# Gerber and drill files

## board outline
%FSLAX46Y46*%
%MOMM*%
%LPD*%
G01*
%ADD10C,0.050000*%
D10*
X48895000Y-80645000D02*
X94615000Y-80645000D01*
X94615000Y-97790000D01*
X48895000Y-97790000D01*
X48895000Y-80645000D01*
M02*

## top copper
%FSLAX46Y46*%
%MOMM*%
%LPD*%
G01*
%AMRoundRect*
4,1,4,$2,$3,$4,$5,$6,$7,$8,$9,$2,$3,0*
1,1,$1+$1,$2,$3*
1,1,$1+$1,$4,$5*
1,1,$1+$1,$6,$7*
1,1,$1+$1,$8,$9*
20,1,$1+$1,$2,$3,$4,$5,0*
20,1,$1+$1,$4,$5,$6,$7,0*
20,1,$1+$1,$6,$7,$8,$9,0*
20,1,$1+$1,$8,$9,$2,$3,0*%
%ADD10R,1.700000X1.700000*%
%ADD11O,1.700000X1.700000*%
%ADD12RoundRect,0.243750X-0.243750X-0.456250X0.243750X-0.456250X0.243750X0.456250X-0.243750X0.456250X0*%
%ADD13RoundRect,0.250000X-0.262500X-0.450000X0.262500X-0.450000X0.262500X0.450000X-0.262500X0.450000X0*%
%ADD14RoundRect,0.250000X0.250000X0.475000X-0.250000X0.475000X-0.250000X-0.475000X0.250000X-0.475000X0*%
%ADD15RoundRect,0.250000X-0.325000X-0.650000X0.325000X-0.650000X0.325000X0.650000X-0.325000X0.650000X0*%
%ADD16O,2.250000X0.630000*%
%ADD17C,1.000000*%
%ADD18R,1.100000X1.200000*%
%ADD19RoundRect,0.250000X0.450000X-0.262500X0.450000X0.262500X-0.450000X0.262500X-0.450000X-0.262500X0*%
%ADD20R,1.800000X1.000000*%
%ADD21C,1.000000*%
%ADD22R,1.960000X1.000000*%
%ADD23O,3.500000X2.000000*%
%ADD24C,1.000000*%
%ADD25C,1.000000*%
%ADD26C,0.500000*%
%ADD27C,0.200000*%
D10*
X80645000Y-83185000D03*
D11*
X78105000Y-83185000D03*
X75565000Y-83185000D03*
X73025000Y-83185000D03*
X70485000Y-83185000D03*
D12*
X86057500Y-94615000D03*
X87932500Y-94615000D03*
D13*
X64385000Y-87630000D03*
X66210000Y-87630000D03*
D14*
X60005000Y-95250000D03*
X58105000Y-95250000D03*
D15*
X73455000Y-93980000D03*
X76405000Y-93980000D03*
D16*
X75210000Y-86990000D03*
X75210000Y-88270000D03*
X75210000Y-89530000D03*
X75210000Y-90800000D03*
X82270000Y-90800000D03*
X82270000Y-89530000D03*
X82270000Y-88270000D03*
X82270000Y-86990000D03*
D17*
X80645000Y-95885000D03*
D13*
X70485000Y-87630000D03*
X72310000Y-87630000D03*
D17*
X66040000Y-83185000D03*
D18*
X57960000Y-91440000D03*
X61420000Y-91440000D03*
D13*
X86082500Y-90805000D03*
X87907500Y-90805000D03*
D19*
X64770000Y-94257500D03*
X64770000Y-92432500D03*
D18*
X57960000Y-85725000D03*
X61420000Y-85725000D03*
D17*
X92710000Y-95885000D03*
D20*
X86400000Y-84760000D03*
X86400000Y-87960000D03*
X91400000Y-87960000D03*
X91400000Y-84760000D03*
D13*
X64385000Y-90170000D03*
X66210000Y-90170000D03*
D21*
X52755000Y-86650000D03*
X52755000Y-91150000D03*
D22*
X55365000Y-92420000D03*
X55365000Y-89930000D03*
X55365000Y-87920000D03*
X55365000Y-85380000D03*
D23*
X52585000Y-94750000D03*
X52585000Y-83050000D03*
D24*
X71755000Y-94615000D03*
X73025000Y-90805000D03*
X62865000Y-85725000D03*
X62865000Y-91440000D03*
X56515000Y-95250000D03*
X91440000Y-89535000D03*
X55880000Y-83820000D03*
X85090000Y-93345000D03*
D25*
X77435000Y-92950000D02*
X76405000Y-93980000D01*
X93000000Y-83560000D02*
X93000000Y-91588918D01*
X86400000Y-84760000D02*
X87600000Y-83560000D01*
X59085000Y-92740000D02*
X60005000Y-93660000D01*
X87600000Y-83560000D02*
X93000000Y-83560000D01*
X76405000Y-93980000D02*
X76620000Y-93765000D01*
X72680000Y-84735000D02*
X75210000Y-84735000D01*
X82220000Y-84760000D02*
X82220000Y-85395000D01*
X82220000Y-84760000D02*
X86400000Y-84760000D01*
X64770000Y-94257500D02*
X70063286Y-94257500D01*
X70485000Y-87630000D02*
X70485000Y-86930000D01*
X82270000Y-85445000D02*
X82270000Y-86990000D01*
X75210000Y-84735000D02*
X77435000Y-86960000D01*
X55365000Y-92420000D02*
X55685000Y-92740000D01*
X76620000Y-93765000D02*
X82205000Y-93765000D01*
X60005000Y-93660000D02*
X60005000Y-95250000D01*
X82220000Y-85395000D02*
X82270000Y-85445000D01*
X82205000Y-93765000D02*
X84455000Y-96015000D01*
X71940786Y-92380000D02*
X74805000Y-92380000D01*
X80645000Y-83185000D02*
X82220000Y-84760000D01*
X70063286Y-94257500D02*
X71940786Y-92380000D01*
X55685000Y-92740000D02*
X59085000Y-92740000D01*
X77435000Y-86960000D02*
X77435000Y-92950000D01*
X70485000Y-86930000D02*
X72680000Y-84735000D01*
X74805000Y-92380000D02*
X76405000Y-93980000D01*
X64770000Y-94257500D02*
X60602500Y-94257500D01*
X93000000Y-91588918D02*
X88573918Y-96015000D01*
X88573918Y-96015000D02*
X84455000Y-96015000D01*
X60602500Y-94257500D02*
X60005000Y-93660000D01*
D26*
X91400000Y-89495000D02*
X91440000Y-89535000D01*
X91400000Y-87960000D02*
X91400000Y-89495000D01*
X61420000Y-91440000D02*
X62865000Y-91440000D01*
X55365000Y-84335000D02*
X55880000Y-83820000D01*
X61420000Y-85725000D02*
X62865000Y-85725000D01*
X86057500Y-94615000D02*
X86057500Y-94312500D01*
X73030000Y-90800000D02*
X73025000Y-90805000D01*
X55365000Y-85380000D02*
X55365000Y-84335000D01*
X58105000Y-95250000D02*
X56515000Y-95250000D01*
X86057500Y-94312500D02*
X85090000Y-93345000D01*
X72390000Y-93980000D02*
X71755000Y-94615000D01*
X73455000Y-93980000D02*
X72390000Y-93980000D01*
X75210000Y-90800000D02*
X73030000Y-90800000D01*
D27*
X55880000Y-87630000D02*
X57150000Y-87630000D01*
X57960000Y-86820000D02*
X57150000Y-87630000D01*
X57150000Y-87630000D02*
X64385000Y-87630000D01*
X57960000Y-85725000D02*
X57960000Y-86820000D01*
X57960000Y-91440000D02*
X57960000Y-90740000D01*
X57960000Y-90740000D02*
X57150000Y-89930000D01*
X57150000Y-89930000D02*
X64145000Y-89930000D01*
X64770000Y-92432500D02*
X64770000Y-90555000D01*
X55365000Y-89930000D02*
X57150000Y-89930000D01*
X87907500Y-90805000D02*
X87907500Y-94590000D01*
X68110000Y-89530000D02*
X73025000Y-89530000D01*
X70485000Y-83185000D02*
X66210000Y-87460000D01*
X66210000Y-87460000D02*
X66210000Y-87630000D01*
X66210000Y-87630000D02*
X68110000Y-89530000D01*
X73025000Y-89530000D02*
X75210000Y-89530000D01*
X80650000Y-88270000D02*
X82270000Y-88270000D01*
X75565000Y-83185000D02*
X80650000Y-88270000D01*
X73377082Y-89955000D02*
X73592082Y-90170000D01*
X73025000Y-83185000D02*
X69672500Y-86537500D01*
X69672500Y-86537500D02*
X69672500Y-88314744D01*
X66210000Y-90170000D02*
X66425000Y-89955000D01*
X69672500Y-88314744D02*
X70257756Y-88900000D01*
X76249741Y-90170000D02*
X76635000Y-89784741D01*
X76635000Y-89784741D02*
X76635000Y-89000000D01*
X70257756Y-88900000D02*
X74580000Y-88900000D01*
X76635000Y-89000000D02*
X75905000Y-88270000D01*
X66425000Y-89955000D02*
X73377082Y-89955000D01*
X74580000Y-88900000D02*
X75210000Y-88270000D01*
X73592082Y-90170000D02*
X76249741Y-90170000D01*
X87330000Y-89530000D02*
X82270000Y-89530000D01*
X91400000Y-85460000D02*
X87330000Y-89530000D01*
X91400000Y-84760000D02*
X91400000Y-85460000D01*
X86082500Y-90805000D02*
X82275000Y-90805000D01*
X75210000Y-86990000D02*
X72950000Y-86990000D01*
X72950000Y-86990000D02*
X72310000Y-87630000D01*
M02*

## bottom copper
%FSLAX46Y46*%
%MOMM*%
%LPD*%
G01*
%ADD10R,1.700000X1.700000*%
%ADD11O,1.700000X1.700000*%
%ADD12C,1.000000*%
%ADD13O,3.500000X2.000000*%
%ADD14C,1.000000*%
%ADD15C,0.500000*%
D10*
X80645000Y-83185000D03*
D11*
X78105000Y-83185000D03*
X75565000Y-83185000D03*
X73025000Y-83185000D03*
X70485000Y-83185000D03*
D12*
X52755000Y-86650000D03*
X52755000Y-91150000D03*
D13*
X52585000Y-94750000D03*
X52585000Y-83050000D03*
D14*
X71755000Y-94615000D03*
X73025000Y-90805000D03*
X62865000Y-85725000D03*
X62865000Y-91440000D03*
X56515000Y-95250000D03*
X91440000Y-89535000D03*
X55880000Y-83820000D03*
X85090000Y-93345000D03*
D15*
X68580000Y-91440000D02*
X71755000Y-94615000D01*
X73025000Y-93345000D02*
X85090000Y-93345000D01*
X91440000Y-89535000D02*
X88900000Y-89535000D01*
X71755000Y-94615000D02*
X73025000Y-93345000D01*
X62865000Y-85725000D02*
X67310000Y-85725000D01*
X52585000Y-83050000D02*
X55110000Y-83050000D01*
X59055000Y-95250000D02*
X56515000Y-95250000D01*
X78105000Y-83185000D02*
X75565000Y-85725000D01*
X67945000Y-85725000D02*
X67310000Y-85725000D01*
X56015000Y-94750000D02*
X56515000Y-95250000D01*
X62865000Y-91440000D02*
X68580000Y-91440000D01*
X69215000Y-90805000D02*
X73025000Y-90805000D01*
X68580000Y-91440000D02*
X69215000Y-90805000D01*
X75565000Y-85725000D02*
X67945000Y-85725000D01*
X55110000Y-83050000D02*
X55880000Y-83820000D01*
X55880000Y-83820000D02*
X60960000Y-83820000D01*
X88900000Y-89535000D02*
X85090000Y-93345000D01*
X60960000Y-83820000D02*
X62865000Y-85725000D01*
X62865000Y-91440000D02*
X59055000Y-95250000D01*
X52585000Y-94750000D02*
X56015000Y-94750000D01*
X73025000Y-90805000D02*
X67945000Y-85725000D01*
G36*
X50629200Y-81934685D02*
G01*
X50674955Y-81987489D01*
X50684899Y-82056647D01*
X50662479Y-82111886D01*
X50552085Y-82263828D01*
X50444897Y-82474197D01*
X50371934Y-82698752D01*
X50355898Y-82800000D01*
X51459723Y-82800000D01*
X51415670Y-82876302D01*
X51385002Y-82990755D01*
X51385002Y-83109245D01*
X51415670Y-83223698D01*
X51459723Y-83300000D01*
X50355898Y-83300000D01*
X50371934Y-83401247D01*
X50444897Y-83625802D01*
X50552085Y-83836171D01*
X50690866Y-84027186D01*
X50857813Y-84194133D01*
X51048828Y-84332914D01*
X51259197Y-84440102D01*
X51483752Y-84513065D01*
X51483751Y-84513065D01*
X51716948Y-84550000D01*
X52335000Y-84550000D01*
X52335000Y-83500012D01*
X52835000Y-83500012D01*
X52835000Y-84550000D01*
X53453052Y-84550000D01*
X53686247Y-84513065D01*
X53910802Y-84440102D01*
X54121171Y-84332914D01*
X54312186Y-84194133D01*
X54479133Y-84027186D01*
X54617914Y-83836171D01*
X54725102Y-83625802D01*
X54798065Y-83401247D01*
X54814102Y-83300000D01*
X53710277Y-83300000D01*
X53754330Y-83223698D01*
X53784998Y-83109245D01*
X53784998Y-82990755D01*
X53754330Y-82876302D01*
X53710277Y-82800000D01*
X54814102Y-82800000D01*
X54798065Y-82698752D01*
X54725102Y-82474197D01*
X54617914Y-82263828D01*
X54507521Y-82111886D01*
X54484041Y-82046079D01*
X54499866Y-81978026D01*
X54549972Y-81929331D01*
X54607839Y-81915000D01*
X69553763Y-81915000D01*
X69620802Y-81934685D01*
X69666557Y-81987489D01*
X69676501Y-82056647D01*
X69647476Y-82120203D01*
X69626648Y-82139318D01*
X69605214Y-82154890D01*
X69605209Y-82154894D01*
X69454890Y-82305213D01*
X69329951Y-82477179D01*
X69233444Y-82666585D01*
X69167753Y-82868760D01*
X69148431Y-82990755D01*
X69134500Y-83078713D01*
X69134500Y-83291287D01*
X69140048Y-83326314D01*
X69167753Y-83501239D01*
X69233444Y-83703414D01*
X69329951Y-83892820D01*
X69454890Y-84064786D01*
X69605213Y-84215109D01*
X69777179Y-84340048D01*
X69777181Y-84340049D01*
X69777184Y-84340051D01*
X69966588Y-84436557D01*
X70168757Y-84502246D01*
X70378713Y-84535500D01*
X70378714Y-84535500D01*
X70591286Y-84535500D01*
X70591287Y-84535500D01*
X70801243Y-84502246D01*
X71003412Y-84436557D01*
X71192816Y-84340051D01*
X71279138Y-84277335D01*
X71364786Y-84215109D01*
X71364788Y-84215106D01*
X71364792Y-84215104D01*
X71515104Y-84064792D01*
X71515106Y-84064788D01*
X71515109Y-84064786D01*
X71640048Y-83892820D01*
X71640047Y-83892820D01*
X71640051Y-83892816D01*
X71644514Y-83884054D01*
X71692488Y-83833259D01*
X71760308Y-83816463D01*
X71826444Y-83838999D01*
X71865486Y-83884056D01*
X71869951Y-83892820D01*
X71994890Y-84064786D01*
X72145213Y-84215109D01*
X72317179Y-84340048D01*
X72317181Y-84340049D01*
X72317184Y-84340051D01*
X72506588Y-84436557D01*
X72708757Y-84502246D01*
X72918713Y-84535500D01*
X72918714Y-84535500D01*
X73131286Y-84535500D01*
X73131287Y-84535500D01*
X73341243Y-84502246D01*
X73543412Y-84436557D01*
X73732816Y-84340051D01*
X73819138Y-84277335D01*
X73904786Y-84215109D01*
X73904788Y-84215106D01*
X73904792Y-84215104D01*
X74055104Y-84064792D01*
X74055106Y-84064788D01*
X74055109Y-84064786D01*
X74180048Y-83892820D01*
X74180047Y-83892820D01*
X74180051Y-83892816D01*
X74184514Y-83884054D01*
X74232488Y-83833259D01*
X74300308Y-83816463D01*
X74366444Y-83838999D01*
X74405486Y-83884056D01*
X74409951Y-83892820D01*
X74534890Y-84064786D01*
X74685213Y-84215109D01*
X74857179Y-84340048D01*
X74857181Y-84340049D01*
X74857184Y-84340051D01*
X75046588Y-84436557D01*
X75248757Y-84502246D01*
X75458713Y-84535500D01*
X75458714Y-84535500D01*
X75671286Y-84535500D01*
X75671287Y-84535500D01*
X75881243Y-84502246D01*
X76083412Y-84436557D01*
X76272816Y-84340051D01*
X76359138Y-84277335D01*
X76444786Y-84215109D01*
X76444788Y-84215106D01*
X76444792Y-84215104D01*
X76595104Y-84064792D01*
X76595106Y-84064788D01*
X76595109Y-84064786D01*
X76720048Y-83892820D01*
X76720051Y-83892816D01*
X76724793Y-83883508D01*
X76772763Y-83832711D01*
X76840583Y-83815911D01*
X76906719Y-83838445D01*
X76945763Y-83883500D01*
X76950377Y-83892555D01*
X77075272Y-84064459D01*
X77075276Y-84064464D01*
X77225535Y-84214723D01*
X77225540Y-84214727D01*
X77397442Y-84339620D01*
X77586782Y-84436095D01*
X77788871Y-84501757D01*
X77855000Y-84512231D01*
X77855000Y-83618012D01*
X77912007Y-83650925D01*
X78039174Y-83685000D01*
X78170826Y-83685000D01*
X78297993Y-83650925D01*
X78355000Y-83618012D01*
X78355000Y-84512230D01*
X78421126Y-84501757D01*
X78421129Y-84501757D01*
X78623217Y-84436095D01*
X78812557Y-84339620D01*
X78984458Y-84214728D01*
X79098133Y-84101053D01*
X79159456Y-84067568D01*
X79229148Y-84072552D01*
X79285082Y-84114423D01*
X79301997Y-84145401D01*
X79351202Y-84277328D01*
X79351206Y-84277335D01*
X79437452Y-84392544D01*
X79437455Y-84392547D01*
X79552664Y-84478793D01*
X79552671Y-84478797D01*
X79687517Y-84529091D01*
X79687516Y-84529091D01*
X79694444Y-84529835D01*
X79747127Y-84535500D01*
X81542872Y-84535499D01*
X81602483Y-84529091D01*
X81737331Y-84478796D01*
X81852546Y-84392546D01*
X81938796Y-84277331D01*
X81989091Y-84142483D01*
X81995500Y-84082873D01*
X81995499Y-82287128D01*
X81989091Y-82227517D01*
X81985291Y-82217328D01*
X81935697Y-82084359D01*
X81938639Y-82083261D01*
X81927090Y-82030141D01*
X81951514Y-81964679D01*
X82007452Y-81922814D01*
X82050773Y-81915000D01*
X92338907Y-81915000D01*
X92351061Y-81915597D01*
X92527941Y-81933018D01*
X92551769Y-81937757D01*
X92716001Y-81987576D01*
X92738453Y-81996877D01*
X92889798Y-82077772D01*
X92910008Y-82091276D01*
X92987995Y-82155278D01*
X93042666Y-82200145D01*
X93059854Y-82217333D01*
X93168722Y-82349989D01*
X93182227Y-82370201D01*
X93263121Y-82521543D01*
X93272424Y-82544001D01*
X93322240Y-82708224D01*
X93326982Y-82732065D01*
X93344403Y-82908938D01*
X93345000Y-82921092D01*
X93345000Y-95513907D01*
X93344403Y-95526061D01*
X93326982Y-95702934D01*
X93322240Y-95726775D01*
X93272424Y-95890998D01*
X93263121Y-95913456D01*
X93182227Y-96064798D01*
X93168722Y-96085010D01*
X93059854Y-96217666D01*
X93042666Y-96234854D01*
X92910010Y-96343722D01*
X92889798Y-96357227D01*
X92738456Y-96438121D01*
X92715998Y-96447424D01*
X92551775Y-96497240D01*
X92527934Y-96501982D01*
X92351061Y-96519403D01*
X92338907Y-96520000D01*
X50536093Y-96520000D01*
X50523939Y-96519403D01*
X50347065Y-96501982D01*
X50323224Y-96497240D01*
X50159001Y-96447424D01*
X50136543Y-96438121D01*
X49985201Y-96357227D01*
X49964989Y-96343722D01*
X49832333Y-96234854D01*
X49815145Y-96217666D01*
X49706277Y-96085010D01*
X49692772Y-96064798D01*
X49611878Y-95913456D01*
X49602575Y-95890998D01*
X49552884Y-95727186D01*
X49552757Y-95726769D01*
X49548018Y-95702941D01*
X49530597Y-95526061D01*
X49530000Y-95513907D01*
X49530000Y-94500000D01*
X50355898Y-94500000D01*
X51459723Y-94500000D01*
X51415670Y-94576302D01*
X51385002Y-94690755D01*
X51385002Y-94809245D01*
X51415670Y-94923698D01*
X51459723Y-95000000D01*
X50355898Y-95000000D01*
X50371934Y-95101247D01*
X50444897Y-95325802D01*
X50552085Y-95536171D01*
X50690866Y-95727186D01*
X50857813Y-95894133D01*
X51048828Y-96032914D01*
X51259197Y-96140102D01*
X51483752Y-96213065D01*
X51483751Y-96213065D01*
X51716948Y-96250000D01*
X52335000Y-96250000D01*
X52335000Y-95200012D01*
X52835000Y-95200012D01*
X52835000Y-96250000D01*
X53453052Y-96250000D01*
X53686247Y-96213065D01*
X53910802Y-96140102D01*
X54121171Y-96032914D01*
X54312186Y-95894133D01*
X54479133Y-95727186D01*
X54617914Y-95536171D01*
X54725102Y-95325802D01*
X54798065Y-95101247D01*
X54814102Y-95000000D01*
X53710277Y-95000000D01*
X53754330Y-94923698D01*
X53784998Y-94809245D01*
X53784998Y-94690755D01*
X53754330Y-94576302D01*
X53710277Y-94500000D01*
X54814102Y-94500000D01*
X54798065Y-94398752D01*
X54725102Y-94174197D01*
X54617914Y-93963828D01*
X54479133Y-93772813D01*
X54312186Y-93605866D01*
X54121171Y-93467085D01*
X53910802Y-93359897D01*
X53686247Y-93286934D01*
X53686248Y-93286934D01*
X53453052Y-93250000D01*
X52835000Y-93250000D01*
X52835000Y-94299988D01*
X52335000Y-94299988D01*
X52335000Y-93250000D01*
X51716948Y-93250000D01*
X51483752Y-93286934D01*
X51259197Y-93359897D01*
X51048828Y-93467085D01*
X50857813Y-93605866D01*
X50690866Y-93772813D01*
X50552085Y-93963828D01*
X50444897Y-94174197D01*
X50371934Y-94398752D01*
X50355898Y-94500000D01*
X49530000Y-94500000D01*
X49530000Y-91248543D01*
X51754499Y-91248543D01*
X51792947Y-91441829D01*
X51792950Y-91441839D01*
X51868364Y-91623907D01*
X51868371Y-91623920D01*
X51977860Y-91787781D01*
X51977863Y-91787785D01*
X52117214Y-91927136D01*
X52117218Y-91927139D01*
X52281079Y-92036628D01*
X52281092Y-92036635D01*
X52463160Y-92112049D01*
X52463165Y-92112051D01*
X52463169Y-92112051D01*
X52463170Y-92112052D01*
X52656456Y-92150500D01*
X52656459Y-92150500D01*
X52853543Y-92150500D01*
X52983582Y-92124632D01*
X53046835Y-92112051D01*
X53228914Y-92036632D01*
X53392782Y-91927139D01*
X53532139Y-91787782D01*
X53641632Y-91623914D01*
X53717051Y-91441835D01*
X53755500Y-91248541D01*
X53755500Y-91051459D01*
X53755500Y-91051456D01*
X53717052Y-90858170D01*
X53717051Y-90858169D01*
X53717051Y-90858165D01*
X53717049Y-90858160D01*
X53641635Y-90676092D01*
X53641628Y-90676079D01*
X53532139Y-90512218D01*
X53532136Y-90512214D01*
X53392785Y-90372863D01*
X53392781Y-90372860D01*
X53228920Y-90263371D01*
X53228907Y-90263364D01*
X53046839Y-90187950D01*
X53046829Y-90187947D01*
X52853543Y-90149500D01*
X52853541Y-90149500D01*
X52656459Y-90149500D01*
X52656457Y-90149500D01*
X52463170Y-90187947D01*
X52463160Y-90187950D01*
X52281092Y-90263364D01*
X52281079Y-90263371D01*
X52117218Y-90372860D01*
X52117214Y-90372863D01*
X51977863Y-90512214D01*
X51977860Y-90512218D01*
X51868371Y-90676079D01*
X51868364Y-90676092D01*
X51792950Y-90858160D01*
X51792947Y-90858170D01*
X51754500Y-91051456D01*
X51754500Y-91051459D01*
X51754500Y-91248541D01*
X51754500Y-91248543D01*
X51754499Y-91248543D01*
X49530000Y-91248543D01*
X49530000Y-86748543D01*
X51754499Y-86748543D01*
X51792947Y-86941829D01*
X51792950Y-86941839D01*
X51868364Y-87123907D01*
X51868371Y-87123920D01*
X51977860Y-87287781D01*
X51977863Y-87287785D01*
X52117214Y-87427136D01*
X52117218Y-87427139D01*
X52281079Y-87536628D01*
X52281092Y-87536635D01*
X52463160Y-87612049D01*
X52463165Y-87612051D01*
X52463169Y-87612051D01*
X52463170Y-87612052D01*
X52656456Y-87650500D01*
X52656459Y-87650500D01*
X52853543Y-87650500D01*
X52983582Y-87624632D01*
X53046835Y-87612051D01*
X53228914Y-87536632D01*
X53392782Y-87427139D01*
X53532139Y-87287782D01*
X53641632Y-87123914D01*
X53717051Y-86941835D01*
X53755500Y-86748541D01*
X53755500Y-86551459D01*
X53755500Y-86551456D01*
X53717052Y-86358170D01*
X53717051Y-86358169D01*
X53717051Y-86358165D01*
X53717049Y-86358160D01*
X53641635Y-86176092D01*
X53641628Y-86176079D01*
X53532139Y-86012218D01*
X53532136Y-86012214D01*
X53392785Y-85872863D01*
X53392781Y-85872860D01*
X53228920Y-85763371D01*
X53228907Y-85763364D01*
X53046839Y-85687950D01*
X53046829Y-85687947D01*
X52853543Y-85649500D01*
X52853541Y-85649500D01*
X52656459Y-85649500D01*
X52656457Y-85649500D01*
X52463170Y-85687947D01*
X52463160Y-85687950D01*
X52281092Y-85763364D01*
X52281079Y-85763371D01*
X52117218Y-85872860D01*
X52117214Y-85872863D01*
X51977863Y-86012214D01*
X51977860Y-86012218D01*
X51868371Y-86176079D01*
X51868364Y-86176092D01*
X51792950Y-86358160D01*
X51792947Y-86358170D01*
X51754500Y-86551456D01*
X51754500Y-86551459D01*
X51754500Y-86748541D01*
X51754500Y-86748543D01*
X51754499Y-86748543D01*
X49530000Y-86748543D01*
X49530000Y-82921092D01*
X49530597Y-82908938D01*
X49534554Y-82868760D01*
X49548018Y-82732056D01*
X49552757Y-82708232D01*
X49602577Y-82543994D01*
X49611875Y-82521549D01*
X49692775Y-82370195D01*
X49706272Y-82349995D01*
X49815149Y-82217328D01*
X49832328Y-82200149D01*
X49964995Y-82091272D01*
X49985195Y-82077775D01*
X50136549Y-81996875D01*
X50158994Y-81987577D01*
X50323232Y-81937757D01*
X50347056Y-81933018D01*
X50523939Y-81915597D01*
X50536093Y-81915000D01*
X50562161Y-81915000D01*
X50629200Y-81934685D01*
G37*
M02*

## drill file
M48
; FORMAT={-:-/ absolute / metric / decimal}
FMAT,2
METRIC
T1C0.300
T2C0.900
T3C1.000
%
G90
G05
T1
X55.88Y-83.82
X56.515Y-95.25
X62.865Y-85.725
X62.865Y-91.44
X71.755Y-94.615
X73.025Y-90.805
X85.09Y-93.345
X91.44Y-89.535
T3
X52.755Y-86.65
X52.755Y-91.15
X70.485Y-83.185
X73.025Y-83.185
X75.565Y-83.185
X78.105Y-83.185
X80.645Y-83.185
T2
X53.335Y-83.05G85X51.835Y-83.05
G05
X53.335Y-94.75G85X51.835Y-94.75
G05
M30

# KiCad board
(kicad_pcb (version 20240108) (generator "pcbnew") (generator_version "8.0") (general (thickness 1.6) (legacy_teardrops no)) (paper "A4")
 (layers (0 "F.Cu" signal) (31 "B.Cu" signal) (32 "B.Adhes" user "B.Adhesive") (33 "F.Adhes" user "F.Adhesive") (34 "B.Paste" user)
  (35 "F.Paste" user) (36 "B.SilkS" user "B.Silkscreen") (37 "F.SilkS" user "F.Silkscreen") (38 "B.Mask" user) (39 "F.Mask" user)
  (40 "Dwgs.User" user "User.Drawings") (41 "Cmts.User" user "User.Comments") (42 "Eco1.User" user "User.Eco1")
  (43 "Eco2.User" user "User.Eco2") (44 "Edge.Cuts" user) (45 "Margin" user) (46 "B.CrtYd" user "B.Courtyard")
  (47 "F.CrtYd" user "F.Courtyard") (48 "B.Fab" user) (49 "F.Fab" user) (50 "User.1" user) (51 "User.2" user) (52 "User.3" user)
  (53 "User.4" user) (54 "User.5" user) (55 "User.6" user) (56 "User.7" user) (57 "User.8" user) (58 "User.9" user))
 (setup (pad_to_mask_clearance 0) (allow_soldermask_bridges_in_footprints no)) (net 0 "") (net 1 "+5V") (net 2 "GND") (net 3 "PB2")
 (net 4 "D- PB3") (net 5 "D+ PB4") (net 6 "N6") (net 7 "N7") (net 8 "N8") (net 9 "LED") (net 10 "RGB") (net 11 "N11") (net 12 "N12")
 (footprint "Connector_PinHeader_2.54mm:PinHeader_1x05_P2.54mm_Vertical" (layer "F.Cu") (at 80.645 83.185 -90)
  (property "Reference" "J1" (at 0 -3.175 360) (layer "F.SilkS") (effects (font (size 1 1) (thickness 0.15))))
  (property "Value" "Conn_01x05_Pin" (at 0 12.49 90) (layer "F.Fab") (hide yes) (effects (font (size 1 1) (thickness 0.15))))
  (pad "1" thru_hole rect (at 0 0 270) (size 1.7 1.7) (drill 1) (layers "*.Cu" "*.Mask") (remove_unused_layers no) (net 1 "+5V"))
  (pad "2" thru_hole oval (at 0 2.54 270) (size 1.7 1.7) (drill 1) (layers "*.Cu" "*.Mask") (remove_unused_layers no) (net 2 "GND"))
  (pad "3" thru_hole oval (at 0 5.08 270) (size 1.7 1.7) (drill 1) (layers "*.Cu" "*.Mask") (remove_unused_layers no) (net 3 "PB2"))
  (pad "4" thru_hole oval (at 0 7.62 270) (size 1.7 1.7) (drill 1) (layers "*.Cu" "*.Mask") (remove_unused_layers no) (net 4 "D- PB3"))
  (pad "5" thru_hole oval (at 0 10.16 270) (size 1.7 1.7) (drill 1) (layers "*.Cu" "*.Mask") (remove_unused_layers no) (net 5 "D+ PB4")))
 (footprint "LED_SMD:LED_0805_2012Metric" (layer "F.Cu") (at 86.995 94.615)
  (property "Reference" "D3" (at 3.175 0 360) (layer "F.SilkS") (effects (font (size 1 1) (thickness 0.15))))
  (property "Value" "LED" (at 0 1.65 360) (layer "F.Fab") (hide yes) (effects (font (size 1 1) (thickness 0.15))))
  (pad "1" smd roundrect (at -0.9375 0) (size 0.975 1.4) (layers "F.Cu" "F.Paste" "F.Mask") (roundrect_rratio 0.25) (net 2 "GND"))
  (pad "2" smd roundrect (at 0.9375 0) (size 0.975 1.4) (layers "F.Cu" "F.Paste" "F.Mask") (roundrect_rratio 0.25) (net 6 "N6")))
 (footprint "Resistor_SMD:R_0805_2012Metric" (layer "F.Cu") (at 65.2975 87.63)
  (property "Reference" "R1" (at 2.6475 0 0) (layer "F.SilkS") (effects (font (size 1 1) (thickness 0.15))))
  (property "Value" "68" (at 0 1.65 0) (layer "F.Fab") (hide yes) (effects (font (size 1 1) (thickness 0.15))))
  (pad "1" smd roundrect (at -0.9125 0) (size 1.025 1.4) (layers "F.Cu" "F.Paste" "F.Mask") (roundrect_rratio 0.243902) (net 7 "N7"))
  (pad "2" smd roundrect (at 0.9125 0) (size 1.025 1.4) (layers "F.Cu" "F.Paste" "F.Mask") (roundrect_rratio 0.243902) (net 5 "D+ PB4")))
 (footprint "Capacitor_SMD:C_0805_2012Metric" (layer "F.Cu") (at 59.055 95.25 180)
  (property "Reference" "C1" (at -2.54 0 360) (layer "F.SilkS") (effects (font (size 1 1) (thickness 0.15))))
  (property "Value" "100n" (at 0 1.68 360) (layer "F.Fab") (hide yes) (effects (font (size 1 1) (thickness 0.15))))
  (pad "1" smd roundrect (at -0.95 0 180) (size 1 1.45) (layers "F.Cu" "F.Paste" "F.Mask") (roundrect_rratio 0.25) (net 1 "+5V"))
  (pad "2" smd roundrect (at 0.95 0 180) (size 1 1.45) (layers "F.Cu" "F.Paste" "F.Mask") (roundrect_rratio 0.25) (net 2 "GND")))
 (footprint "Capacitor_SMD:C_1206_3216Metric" (layer "F.Cu") (at 74.93 93.98)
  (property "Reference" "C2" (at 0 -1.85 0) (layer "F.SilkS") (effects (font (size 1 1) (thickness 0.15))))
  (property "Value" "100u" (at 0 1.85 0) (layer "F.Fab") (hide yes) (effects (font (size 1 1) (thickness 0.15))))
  (pad "1" smd roundrect (at -1.475 0) (size 1.15 1.8) (layers "F.Cu" "F.Paste" "F.Mask") (roundrect_rratio 0.217391) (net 2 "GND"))
  (pad "2" smd roundrect (at 1.475 0) (size 1.15 1.8) (layers "F.Cu" "F.Paste" "F.Mask") (roundrect_rratio 0.217391) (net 1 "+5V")))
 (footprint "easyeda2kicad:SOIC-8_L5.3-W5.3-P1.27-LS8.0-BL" (layer "F.Cu") (at 78.74 88.9 -90)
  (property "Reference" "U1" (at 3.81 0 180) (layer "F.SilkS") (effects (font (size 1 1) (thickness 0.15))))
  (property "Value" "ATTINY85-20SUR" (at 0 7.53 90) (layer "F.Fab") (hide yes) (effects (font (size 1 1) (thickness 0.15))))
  (pad "1" smd oval (at -1.91 3.53 270) (size 0.63 2.25) (layers "F.Cu" "F.Paste" "F.Mask") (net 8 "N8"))
  (pad "2" smd oval (at -0.63 3.53 270) (size 0.63 2.25) (layers "F.Cu" "F.Paste" "F.Mask") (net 4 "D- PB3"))
  (pad "3" smd oval (at 0.63 3.53 270) (size 0.63 2.25) (layers "F.Cu" "F.Paste" "F.Mask") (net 5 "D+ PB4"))
  (pad "4" smd oval (at 1.9 3.53 270) (size 0.63 2.25) (layers "F.Cu" "F.Paste" "F.Mask") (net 2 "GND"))
  (pad "5" smd oval (at 1.9 -3.53 270) (size 0.63 2.25) (layers "F.Cu" "F.Paste" "F.Mask") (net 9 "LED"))
  (pad "6" smd oval (at 0.63 -3.53 270) (size 0.63 2.25) (layers "F.Cu" "F.Paste" "F.Mask") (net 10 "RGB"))
  (pad "7" smd oval (at -0.63 -3.53 270) (size 0.63 2.25) (layers "F.Cu" "F.Paste" "F.Mask") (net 3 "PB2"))
  (pad "8" smd oval (at -1.91 -3.53 270) (size 0.63 2.25) (layers "F.Cu" "F.Paste" "F.Mask") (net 1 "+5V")))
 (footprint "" (layer "F.Cu") (at 80.645 95.885)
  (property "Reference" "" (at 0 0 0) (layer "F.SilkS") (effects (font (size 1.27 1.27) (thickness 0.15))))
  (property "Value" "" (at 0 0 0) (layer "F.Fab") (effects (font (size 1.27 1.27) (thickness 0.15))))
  (pad "" smd circle (at 0 0) (size 1 1) (layers "F.Cu" "F.Mask") (solder_mask_margin 1) (clearance 1)))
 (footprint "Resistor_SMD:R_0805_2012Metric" (layer "F.Cu") (at 71.3975 87.63)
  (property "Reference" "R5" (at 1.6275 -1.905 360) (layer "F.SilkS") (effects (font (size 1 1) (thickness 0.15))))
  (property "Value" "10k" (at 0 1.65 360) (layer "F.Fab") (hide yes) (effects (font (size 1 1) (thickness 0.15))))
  (pad "1" smd roundrect (at -0.9125 0) (size 1.025 1.4) (layers "F.Cu" "F.Paste" "F.Mask") (roundrect_rratio 0.243902) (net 1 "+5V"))
  (pad "2" smd roundrect (at 0.9125 0) (size 1.025 1.4) (layers "F.Cu" "F.Paste" "F.Mask") (roundrect_rratio 0.243902) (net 8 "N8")))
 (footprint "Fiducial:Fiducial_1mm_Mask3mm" (layer "F.Cu") (at 66.04 83.185)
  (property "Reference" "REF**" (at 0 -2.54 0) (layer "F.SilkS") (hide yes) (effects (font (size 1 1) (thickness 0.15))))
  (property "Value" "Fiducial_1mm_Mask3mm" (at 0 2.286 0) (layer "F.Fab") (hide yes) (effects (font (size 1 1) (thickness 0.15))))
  (pad "" smd circle (at 0 0) (size 1 1) (layers "F.Cu" "F.Mask") (solder_mask_margin 1) (clearance 1)))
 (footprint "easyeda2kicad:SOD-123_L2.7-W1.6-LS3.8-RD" (layer "F.Cu") (at 59.69 91.44)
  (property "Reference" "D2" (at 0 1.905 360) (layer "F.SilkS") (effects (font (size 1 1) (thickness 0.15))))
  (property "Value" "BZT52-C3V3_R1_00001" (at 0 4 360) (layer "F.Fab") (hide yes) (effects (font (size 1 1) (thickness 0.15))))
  (pad "1" smd rect (at -1.73 0) (size 1.1 1.2) (layers "F.Cu" "F.Paste" "F.Mask") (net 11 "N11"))
  (pad "2" smd rect (at 1.73 0) (size 1.1 1.2) (layers "F.Cu" "F.Paste" "F.Mask") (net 2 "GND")))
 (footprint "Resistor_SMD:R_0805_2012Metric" (layer "F.Cu") (at 86.995 90.805)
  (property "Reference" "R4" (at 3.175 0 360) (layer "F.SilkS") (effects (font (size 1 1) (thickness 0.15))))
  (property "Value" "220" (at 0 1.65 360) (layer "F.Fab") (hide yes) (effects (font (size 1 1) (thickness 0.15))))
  (pad "1" smd roundrect (at -0.9125 0) (size 1.025 1.4) (layers "F.Cu" "F.Paste" "F.Mask") (roundrect_rratio 0.243902) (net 9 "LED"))
  (pad "2" smd roundrect (at 0.9125 0) (size 1.025 1.4) (layers "F.Cu" "F.Paste" "F.Mask") (roundrect_rratio 0.243902) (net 6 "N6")))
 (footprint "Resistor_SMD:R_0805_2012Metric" (layer "F.Cu") (at 64.77 93.345 90)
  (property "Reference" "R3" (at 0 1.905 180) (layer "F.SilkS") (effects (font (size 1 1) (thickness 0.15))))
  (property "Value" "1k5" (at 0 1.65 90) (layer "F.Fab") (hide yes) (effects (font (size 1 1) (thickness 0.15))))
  (pad "1" smd roundrect (at -0.9125 0 90) (size 1.025 1.4) (layers "F.Cu" "F.Paste" "F.Mask") (roundrect_rratio 0.243902) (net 1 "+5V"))
  (pad "2" smd roundrect (at 0.9125 0 90) (size 1.025 1.4) (layers "F.Cu" "F.Paste" "F.Mask") (roundrect_rratio 0.243902) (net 11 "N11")))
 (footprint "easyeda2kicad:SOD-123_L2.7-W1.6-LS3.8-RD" (layer "F.Cu") (at 59.69 85.725)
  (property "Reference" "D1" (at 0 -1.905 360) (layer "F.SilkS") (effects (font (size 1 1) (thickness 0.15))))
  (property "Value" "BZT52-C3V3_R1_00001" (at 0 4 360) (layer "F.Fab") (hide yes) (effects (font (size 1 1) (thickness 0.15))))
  (pad "1" smd rect (at -1.73 0) (size 1.1 1.2) (layers "F.Cu" "F.Paste" "F.Mask") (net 7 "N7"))
  (pad "2" smd rect (at 1.73 0) (size 1.1 1.2) (layers "F.Cu" "F.Paste" "F.Mask") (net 2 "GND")))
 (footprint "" (layer "F.Cu") (at 92.71 95.885)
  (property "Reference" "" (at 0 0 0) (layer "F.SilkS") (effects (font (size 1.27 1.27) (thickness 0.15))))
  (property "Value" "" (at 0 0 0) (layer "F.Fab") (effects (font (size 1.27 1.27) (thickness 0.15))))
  (pad "" smd circle (at 0 0) (size 1 1) (layers "F.Cu" "F.Mask") (solder_mask_margin 1) (clearance 1)))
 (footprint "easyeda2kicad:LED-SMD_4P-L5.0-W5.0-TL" (layer "F.Cu") (at 88.9 86.36)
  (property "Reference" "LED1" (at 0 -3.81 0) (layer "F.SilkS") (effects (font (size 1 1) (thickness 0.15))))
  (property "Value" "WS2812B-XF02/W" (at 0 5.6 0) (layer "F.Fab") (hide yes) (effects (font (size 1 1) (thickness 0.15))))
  (pad "1" smd rect (at -2.5 -1.6 180) (size 1.8 1) (layers "F.Cu" "F.Paste" "F.Mask") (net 1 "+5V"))
  (pad "2" smd rect (at -2.5 1.6 180) (size 1.8 1) (layers "F.Cu" "F.Paste" "F.Mask") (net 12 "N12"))
  (pad "3" smd rect (at 2.5 1.6 180) (size 1.8 1) (layers "F.Cu" "F.Paste" "F.Mask") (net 2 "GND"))
  (pad "4" smd rect (at 2.5 -1.6 180) (size 1.8 1) (layers "F.Cu" "F.Paste" "F.Mask") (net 10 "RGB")))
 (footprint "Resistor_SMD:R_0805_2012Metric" (layer "F.Cu") (at 65.2975 90.17)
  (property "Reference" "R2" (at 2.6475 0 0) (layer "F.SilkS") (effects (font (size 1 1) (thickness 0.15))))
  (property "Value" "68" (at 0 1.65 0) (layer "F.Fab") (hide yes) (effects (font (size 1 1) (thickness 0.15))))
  (pad "1" smd roundrect (at -0.9125 0) (size 1.025 1.4) (layers "F.Cu" "F.Paste" "F.Mask") (roundrect_rratio 0.243902) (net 11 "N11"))
  (pad "2" smd roundrect (at 0.9125 0) (size 1.025 1.4) (layers "F.Cu" "F.Paste" "F.Mask") (roundrect_rratio 0.243902) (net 4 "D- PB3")))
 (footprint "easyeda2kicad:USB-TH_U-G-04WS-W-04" (layer "F.Cu") (at 53.975 88.9 -90)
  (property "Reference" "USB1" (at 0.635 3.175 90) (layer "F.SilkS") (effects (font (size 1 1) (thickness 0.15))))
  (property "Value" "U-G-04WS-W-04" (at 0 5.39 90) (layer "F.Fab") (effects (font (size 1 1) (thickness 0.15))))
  (pad "" thru_hole circle (at -2.25 1.22 270) (size 1 1) (drill 1) (layers "*.Cu" "*.Mask") (remove_unused_layers no))
  (pad "" thru_hole circle (at 2.25 1.22 270) (size 1 1) (drill 1) (layers "*.Cu" "*.Mask") (remove_unused_layers no))
  (pad "1" smd rect (at 3.52 -1.39 180) (size 1.96 1) (layers "F.Cu" "F.Paste" "F.Mask") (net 1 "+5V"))
  (pad "2" smd rect (at 1.03 -1.39 180) (size 1.96 1) (layers "F.Cu" "F.Paste" "F.Mask") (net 11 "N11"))
  (pad "3" smd rect (at -0.98 -1.39 180) (size 1.96 1) (layers "F.Cu" "F.Paste" "F.Mask") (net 7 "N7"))
  (pad "4" smd rect (at -3.52 -1.39 180) (size 1.96 1) (layers "F.Cu" "F.Paste" "F.Mask") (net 2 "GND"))
  (pad "5" thru_hole oval (at 5.85 1.39 180) (size 3.5 2) (drill oval 2.399995 0.900024) (layers "*.Cu" "*.Mask") (remove_unused_layers no)
   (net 2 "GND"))
  (pad "6" thru_hole oval (at -5.85 1.39 180) (size 3.5 2) (drill oval 2.399995 0.900024) (layers "*.Cu" "*.Mask") (remove_unused_layers no)
   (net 2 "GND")))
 (gr_poly
  (pts (xy 48.895 80.645) (xy 94.615 80.645) (xy 94.615 97.79) (xy 48.895 97.79)) (stroke (width 0.05) (type solid)) (fill none)
  (layer "Edge.Cuts"))
 (segment (start 77.435 92.95) (end 76.405 93.98) (width 1) (layer "F.Cu") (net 1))
 (segment (start 93 83.56) (end 93 91.588918) (width 1) (layer "F.Cu") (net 1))
 (segment (start 86.4 84.76) (end 87.6 83.56) (width 1) (layer "F.Cu") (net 1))
 (segment (start 59.085 92.74) (end 60.005 93.66) (width 1) (layer "F.Cu") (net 1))
 (segment (start 87.6 83.56) (end 93 83.56) (width 1) (layer "F.Cu") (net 1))
 (segment (start 76.405 93.98) (end 76.62 93.765) (width 1) (layer "F.Cu") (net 1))
 (segment (start 72.68 84.735) (end 75.21 84.735) (width 1) (layer "F.Cu") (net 1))
 (segment (start 82.22 84.76) (end 82.22 85.395) (width 1) (layer "F.Cu") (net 1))
 (segment (start 82.22 84.76) (end 86.4 84.76) (width 1) (layer "F.Cu") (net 1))
 (segment (start 64.77 94.2575) (end 70.063286 94.2575) (width 1) (layer "F.Cu") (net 1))
 (segment (start 70.485 87.63) (end 70.485 86.93) (width 1) (layer "F.Cu") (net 1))
 (segment (start 82.27 85.445) (end 82.27 86.99) (width 1) (layer "F.Cu") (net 1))
 (segment (start 75.21 84.735) (end 77.435 86.96) (width 1) (layer "F.Cu") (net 1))
 (segment (start 55.365 92.42) (end 55.685 92.74) (width 1) (layer "F.Cu") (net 1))
 (segment (start 76.62 93.765) (end 82.205 93.765) (width 1) (layer "F.Cu") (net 1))
 (segment (start 60.005 93.66) (end 60.005 95.25) (width 1) (layer "F.Cu") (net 1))
 (segment (start 82.22 85.395) (end 82.27 85.445) (width 1) (layer "F.Cu") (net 1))
 (segment (start 82.205 93.765) (end 84.455 96.015) (width 1) (layer "F.Cu") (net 1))
 (segment (start 71.940786 92.38) (end 74.805 92.38) (width 1) (layer "F.Cu") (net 1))
 (segment (start 80.645 83.185) (end 82.22 84.76) (width 1) (layer "F.Cu") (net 1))
 (segment (start 70.063286 94.2575) (end 71.940786 92.38) (width 1) (layer "F.Cu") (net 1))
 (segment (start 55.685 92.74) (end 59.085 92.74) (width 1) (layer "F.Cu") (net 1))
 (segment (start 77.435 86.96) (end 77.435 92.95) (width 1) (layer "F.Cu") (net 1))
 (segment (start 70.485 86.93) (end 72.68 84.735) (width 1) (layer "F.Cu") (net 1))
 (segment (start 74.805 92.38) (end 76.405 93.98) (width 1) (layer "F.Cu") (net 1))
 (segment (start 64.77 94.2575) (end 60.6025 94.2575) (width 1) (layer "F.Cu") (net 1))
 (segment (start 93 91.588918) (end 88.573918 96.015) (width 1) (layer "F.Cu") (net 1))
 (segment (start 88.573918 96.015) (end 84.455 96.015) (width 1) (layer "F.Cu") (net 1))
 (segment (start 60.6025 94.2575) (end 60.005 93.66) (width 1) (layer "F.Cu") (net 1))
 (segment (start 91.4 89.495) (end 91.44 89.535) (width 0.5) (layer "F.Cu") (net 2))
 (segment (start 91.4 87.96) (end 91.4 89.495) (width 0.5) (layer "F.Cu") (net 2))
 (segment (start 61.42 91.44) (end 62.865 91.44) (width 0.5) (layer "F.Cu") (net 2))
 (segment (start 55.365 84.335) (end 55.88 83.82) (width 0.5) (layer "F.Cu") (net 2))
 (segment (start 61.42 85.725) (end 62.865 85.725) (width 0.5) (layer "F.Cu") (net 2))
 (segment (start 86.0575 94.615) (end 86.0575 94.3125) (width 0.5) (layer "F.Cu") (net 2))
 (segment (start 73.03 90.8) (end 73.025 90.805) (width 0.5) (layer "F.Cu") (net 2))
 (segment (start 55.365 85.38) (end 55.365 84.335) (width 0.5) (layer "F.Cu") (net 2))
 (segment (start 58.105 95.25) (end 56.515 95.25) (width 0.5) (layer "F.Cu") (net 2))
 (segment (start 86.0575 94.3125) (end 85.09 93.345) (width 0.5) (layer "F.Cu") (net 2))
 (segment (start 72.39 93.98) (end 71.755 94.615) (width 0.5) (layer "F.Cu") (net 2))
 (segment (start 73.455 93.98) (end 72.39 93.98) (width 0.5) (layer "F.Cu") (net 2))
 (segment (start 75.21 90.8) (end 73.03 90.8) (width 0.5) (layer "F.Cu") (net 2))
 (via (at 71.755 94.615) (size 1) (drill 0.3) (layers "F.Cu" "B.Cu") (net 2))
 (via (at 73.025 90.805) (size 1) (drill 0.3) (layers "F.Cu" "B.Cu") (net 2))
 (via (at 62.865 85.725) (size 1) (drill 0.3) (layers "F.Cu" "B.Cu") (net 2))
 (via (at 62.865 91.44) (size 1) (drill 0.3) (layers "F.Cu" "B.Cu") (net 2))
 (via (at 56.515 95.25) (size 1) (drill 0.3) (layers "F.Cu" "B.Cu") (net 2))
 (via (at 91.44 89.535) (size 1) (drill 0.3) (layers "F.Cu" "B.Cu") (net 2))
 (via (at 55.88 83.82) (size 1) (drill 0.3) (layers "F.Cu" "B.Cu") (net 2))
 (via (at 85.09 93.345) (size 1) (drill 0.3) (layers "F.Cu" "B.Cu") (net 2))
 (segment (start 68.58 91.44) (end 71.755 94.615) (width 0.5) (layer "B.Cu") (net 2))
 (segment (start 73.025 93.345) (end 85.09 93.345) (width 0.5) (layer "B.Cu") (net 2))
 (segment (start 91.44 89.535) (end 88.9 89.535) (width 0.5) (layer "B.Cu") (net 2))
 (segment (start 71.755 94.615) (end 73.025 93.345) (width 0.5) (layer "B.Cu") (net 2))
 (segment (start 62.865 85.725) (end 67.31 85.725) (width 0.5) (layer "B.Cu") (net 2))
 (segment (start 52.585 83.05) (end 55.11 83.05) (width 0.5) (layer "B.Cu") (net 2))
 (segment (start 59.055 95.25) (end 56.515 95.25) (width 0.5) (layer "B.Cu") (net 2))
 (segment (start 78.105 83.185) (end 75.565 85.725) (width 0.5) (layer "B.Cu") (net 2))
 (segment (start 67.945 85.725) (end 67.31 85.725) (width 0.5) (layer "B.Cu") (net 2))
 (segment (start 56.015 94.75) (end 56.515 95.25) (width 0.5) (layer "B.Cu") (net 2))
 (segment (start 62.865 91.44) (end 68.58 91.44) (width 0.5) (layer "B.Cu") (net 2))
 (segment (start 69.215 90.805) (end 73.025 90.805) (width 0.5) (layer "B.Cu") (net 2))
 (segment (start 68.58 91.44) (end 69.215 90.805) (width 0.5) (layer "B.Cu") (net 2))
 (segment (start 75.565 85.725) (end 67.945 85.725) (width 0.5) (layer "B.Cu") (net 2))
 (segment (start 55.11 83.05) (end 55.88 83.82) (width 0.5) (layer "B.Cu") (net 2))
 (segment (start 55.88 83.82) (end 60.96 83.82) (width 0.5) (layer "B.Cu") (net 2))
 (segment (start 88.9 89.535) (end 85.09 93.345) (width 0.5) (layer "B.Cu") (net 2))
 (segment (start 60.96 83.82) (end 62.865 85.725) (width 0.5) (layer "B.Cu") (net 2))
 (segment (start 62.865 91.44) (end 59.055 95.25) (width 0.5) (layer "B.Cu") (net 2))
 (segment (start 52.585 94.75) (end 56.015 94.75) (width 0.5) (layer "B.Cu") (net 2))
 (segment (start 73.025 90.805) (end 67.945 85.725) (width 0.5) (layer "B.Cu") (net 2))
 (segment (start 55.88 87.63) (end 57.15 87.63) (width 0.2) (layer "F.Cu") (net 7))
 (segment (start 57.96 86.82) (end 57.15 87.63) (width 0.2) (layer "F.Cu") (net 7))
 (segment (start 57.15 87.63) (end 64.385 87.63) (width 0.2) (layer "F.Cu") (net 7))
 (segment (start 57.96 85.725) (end 57.96 86.82) (width 0.2) (layer "F.Cu") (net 7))
 (segment (start 57.96 91.44) (end 57.96 90.74) (width 0.2) (layer "F.Cu") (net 11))
 (segment (start 57.96 90.74) (end 57.15 89.93) (width 0.2) (layer "F.Cu") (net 11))
 (segment (start 57.15 89.93) (end 64.145 89.93) (width 0.2) (layer "F.Cu") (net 11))
 (segment (start 64.77 92.4325) (end 64.77 90.555) (width 0.2) (layer "F.Cu") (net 11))
 (segment (start 55.365 89.93) (end 57.15 89.93) (width 0.2) (layer "F.Cu") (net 11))
 (segment (start 87.9075 90.805) (end 87.9075 94.59) (width 0.2) (layer "F.Cu") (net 6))
 (segment (start 68.11 89.53) (end 73.025 89.53) (width 0.2) (layer "F.Cu") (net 5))
 (segment (start 70.485 83.185) (end 66.21 87.46) (width 0.2) (layer "F.Cu") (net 5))
 (segment (start 66.21 87.46) (end 66.21 87.63) (width 0.2) (layer "F.Cu") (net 5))
 (segment (start 66.21 87.63) (end 68.11 89.53) (width 0.2) (layer "F.Cu") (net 5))
 (segment (start 73.025 89.53) (end 75.21 89.53) (width 0.2) (layer "F.Cu") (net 5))
 (segment (start 80.65 88.27) (end 82.27 88.27) (width 0.2) (layer "F.Cu") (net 3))
 (segment (start 75.565 83.185) (end 80.65 88.27) (width 0.2) (layer "F.Cu") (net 3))
 (segment (start 73.377082 89.955) (end 73.592082 90.17) (width 0.2) (layer "F.Cu") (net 4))
 (segment (start 73.025 83.185) (end 69.6725 86.5375) (width 0.2) (layer "F.Cu") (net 4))
 (segment (start 69.6725 86.5375) (end 69.6725 88.314744) (width 0.2) (layer "F.Cu") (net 4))
 (segment (start 66.21 90.17) (end 66.425 89.955) (width 0.2) (layer "F.Cu") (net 4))
 (segment (start 69.6725 88.314744) (end 70.257756 88.9) (width 0.2) (layer "F.Cu") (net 4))
 (segment (start 76.249741 90.17) (end 76.635 89.784741) (width 0.2) (layer "F.Cu") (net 4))
 (segment (start 76.635 89.784741) (end 76.635 89) (width 0.2) (layer "F.Cu") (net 4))
 (segment (start 70.257756 88.9) (end 74.58 88.9) (width 0.2) (layer "F.Cu") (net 4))
 (segment (start 76.635 89) (end 75.905 88.27) (width 0.2) (layer "F.Cu") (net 4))
 (segment (start 66.425 89.955) (end 73.377082 89.955) (width 0.2) (layer "F.Cu") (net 4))
 (segment (start 74.58 88.9) (end 75.21 88.27) (width 0.2) (layer "F.Cu") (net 4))
 (segment (start 73.592082 90.17) (end 76.249741 90.17) (width 0.2) (layer "F.Cu") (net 4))
 (segment (start 87.33 89.53) (end 82.27 89.53) (width 0.2) (layer "F.Cu") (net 10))
 (segment (start 91.4 85.46) (end 87.33 89.53) (width 0.2) (layer "F.Cu") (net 10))
 (segment (start 91.4 84.76) (end 91.4 85.46) (width 0.2) (layer "F.Cu") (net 10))
 (segment (start 86.0825 90.805) (end 82.275 90.805) (width 0.2) (layer "F.Cu") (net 9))
 (segment (start 75.21 86.99) (end 72.95 86.99) (width 0.2) (layer "F.Cu") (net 8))
 (segment (start 72.95 86.99) (end 72.31 87.63) (width 0.2) (layer "F.Cu") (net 8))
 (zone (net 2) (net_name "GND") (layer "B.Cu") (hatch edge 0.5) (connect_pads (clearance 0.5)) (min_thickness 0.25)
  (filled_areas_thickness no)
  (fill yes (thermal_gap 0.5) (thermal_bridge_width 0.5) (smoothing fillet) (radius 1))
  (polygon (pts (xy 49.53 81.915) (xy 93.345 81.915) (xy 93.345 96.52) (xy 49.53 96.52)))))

